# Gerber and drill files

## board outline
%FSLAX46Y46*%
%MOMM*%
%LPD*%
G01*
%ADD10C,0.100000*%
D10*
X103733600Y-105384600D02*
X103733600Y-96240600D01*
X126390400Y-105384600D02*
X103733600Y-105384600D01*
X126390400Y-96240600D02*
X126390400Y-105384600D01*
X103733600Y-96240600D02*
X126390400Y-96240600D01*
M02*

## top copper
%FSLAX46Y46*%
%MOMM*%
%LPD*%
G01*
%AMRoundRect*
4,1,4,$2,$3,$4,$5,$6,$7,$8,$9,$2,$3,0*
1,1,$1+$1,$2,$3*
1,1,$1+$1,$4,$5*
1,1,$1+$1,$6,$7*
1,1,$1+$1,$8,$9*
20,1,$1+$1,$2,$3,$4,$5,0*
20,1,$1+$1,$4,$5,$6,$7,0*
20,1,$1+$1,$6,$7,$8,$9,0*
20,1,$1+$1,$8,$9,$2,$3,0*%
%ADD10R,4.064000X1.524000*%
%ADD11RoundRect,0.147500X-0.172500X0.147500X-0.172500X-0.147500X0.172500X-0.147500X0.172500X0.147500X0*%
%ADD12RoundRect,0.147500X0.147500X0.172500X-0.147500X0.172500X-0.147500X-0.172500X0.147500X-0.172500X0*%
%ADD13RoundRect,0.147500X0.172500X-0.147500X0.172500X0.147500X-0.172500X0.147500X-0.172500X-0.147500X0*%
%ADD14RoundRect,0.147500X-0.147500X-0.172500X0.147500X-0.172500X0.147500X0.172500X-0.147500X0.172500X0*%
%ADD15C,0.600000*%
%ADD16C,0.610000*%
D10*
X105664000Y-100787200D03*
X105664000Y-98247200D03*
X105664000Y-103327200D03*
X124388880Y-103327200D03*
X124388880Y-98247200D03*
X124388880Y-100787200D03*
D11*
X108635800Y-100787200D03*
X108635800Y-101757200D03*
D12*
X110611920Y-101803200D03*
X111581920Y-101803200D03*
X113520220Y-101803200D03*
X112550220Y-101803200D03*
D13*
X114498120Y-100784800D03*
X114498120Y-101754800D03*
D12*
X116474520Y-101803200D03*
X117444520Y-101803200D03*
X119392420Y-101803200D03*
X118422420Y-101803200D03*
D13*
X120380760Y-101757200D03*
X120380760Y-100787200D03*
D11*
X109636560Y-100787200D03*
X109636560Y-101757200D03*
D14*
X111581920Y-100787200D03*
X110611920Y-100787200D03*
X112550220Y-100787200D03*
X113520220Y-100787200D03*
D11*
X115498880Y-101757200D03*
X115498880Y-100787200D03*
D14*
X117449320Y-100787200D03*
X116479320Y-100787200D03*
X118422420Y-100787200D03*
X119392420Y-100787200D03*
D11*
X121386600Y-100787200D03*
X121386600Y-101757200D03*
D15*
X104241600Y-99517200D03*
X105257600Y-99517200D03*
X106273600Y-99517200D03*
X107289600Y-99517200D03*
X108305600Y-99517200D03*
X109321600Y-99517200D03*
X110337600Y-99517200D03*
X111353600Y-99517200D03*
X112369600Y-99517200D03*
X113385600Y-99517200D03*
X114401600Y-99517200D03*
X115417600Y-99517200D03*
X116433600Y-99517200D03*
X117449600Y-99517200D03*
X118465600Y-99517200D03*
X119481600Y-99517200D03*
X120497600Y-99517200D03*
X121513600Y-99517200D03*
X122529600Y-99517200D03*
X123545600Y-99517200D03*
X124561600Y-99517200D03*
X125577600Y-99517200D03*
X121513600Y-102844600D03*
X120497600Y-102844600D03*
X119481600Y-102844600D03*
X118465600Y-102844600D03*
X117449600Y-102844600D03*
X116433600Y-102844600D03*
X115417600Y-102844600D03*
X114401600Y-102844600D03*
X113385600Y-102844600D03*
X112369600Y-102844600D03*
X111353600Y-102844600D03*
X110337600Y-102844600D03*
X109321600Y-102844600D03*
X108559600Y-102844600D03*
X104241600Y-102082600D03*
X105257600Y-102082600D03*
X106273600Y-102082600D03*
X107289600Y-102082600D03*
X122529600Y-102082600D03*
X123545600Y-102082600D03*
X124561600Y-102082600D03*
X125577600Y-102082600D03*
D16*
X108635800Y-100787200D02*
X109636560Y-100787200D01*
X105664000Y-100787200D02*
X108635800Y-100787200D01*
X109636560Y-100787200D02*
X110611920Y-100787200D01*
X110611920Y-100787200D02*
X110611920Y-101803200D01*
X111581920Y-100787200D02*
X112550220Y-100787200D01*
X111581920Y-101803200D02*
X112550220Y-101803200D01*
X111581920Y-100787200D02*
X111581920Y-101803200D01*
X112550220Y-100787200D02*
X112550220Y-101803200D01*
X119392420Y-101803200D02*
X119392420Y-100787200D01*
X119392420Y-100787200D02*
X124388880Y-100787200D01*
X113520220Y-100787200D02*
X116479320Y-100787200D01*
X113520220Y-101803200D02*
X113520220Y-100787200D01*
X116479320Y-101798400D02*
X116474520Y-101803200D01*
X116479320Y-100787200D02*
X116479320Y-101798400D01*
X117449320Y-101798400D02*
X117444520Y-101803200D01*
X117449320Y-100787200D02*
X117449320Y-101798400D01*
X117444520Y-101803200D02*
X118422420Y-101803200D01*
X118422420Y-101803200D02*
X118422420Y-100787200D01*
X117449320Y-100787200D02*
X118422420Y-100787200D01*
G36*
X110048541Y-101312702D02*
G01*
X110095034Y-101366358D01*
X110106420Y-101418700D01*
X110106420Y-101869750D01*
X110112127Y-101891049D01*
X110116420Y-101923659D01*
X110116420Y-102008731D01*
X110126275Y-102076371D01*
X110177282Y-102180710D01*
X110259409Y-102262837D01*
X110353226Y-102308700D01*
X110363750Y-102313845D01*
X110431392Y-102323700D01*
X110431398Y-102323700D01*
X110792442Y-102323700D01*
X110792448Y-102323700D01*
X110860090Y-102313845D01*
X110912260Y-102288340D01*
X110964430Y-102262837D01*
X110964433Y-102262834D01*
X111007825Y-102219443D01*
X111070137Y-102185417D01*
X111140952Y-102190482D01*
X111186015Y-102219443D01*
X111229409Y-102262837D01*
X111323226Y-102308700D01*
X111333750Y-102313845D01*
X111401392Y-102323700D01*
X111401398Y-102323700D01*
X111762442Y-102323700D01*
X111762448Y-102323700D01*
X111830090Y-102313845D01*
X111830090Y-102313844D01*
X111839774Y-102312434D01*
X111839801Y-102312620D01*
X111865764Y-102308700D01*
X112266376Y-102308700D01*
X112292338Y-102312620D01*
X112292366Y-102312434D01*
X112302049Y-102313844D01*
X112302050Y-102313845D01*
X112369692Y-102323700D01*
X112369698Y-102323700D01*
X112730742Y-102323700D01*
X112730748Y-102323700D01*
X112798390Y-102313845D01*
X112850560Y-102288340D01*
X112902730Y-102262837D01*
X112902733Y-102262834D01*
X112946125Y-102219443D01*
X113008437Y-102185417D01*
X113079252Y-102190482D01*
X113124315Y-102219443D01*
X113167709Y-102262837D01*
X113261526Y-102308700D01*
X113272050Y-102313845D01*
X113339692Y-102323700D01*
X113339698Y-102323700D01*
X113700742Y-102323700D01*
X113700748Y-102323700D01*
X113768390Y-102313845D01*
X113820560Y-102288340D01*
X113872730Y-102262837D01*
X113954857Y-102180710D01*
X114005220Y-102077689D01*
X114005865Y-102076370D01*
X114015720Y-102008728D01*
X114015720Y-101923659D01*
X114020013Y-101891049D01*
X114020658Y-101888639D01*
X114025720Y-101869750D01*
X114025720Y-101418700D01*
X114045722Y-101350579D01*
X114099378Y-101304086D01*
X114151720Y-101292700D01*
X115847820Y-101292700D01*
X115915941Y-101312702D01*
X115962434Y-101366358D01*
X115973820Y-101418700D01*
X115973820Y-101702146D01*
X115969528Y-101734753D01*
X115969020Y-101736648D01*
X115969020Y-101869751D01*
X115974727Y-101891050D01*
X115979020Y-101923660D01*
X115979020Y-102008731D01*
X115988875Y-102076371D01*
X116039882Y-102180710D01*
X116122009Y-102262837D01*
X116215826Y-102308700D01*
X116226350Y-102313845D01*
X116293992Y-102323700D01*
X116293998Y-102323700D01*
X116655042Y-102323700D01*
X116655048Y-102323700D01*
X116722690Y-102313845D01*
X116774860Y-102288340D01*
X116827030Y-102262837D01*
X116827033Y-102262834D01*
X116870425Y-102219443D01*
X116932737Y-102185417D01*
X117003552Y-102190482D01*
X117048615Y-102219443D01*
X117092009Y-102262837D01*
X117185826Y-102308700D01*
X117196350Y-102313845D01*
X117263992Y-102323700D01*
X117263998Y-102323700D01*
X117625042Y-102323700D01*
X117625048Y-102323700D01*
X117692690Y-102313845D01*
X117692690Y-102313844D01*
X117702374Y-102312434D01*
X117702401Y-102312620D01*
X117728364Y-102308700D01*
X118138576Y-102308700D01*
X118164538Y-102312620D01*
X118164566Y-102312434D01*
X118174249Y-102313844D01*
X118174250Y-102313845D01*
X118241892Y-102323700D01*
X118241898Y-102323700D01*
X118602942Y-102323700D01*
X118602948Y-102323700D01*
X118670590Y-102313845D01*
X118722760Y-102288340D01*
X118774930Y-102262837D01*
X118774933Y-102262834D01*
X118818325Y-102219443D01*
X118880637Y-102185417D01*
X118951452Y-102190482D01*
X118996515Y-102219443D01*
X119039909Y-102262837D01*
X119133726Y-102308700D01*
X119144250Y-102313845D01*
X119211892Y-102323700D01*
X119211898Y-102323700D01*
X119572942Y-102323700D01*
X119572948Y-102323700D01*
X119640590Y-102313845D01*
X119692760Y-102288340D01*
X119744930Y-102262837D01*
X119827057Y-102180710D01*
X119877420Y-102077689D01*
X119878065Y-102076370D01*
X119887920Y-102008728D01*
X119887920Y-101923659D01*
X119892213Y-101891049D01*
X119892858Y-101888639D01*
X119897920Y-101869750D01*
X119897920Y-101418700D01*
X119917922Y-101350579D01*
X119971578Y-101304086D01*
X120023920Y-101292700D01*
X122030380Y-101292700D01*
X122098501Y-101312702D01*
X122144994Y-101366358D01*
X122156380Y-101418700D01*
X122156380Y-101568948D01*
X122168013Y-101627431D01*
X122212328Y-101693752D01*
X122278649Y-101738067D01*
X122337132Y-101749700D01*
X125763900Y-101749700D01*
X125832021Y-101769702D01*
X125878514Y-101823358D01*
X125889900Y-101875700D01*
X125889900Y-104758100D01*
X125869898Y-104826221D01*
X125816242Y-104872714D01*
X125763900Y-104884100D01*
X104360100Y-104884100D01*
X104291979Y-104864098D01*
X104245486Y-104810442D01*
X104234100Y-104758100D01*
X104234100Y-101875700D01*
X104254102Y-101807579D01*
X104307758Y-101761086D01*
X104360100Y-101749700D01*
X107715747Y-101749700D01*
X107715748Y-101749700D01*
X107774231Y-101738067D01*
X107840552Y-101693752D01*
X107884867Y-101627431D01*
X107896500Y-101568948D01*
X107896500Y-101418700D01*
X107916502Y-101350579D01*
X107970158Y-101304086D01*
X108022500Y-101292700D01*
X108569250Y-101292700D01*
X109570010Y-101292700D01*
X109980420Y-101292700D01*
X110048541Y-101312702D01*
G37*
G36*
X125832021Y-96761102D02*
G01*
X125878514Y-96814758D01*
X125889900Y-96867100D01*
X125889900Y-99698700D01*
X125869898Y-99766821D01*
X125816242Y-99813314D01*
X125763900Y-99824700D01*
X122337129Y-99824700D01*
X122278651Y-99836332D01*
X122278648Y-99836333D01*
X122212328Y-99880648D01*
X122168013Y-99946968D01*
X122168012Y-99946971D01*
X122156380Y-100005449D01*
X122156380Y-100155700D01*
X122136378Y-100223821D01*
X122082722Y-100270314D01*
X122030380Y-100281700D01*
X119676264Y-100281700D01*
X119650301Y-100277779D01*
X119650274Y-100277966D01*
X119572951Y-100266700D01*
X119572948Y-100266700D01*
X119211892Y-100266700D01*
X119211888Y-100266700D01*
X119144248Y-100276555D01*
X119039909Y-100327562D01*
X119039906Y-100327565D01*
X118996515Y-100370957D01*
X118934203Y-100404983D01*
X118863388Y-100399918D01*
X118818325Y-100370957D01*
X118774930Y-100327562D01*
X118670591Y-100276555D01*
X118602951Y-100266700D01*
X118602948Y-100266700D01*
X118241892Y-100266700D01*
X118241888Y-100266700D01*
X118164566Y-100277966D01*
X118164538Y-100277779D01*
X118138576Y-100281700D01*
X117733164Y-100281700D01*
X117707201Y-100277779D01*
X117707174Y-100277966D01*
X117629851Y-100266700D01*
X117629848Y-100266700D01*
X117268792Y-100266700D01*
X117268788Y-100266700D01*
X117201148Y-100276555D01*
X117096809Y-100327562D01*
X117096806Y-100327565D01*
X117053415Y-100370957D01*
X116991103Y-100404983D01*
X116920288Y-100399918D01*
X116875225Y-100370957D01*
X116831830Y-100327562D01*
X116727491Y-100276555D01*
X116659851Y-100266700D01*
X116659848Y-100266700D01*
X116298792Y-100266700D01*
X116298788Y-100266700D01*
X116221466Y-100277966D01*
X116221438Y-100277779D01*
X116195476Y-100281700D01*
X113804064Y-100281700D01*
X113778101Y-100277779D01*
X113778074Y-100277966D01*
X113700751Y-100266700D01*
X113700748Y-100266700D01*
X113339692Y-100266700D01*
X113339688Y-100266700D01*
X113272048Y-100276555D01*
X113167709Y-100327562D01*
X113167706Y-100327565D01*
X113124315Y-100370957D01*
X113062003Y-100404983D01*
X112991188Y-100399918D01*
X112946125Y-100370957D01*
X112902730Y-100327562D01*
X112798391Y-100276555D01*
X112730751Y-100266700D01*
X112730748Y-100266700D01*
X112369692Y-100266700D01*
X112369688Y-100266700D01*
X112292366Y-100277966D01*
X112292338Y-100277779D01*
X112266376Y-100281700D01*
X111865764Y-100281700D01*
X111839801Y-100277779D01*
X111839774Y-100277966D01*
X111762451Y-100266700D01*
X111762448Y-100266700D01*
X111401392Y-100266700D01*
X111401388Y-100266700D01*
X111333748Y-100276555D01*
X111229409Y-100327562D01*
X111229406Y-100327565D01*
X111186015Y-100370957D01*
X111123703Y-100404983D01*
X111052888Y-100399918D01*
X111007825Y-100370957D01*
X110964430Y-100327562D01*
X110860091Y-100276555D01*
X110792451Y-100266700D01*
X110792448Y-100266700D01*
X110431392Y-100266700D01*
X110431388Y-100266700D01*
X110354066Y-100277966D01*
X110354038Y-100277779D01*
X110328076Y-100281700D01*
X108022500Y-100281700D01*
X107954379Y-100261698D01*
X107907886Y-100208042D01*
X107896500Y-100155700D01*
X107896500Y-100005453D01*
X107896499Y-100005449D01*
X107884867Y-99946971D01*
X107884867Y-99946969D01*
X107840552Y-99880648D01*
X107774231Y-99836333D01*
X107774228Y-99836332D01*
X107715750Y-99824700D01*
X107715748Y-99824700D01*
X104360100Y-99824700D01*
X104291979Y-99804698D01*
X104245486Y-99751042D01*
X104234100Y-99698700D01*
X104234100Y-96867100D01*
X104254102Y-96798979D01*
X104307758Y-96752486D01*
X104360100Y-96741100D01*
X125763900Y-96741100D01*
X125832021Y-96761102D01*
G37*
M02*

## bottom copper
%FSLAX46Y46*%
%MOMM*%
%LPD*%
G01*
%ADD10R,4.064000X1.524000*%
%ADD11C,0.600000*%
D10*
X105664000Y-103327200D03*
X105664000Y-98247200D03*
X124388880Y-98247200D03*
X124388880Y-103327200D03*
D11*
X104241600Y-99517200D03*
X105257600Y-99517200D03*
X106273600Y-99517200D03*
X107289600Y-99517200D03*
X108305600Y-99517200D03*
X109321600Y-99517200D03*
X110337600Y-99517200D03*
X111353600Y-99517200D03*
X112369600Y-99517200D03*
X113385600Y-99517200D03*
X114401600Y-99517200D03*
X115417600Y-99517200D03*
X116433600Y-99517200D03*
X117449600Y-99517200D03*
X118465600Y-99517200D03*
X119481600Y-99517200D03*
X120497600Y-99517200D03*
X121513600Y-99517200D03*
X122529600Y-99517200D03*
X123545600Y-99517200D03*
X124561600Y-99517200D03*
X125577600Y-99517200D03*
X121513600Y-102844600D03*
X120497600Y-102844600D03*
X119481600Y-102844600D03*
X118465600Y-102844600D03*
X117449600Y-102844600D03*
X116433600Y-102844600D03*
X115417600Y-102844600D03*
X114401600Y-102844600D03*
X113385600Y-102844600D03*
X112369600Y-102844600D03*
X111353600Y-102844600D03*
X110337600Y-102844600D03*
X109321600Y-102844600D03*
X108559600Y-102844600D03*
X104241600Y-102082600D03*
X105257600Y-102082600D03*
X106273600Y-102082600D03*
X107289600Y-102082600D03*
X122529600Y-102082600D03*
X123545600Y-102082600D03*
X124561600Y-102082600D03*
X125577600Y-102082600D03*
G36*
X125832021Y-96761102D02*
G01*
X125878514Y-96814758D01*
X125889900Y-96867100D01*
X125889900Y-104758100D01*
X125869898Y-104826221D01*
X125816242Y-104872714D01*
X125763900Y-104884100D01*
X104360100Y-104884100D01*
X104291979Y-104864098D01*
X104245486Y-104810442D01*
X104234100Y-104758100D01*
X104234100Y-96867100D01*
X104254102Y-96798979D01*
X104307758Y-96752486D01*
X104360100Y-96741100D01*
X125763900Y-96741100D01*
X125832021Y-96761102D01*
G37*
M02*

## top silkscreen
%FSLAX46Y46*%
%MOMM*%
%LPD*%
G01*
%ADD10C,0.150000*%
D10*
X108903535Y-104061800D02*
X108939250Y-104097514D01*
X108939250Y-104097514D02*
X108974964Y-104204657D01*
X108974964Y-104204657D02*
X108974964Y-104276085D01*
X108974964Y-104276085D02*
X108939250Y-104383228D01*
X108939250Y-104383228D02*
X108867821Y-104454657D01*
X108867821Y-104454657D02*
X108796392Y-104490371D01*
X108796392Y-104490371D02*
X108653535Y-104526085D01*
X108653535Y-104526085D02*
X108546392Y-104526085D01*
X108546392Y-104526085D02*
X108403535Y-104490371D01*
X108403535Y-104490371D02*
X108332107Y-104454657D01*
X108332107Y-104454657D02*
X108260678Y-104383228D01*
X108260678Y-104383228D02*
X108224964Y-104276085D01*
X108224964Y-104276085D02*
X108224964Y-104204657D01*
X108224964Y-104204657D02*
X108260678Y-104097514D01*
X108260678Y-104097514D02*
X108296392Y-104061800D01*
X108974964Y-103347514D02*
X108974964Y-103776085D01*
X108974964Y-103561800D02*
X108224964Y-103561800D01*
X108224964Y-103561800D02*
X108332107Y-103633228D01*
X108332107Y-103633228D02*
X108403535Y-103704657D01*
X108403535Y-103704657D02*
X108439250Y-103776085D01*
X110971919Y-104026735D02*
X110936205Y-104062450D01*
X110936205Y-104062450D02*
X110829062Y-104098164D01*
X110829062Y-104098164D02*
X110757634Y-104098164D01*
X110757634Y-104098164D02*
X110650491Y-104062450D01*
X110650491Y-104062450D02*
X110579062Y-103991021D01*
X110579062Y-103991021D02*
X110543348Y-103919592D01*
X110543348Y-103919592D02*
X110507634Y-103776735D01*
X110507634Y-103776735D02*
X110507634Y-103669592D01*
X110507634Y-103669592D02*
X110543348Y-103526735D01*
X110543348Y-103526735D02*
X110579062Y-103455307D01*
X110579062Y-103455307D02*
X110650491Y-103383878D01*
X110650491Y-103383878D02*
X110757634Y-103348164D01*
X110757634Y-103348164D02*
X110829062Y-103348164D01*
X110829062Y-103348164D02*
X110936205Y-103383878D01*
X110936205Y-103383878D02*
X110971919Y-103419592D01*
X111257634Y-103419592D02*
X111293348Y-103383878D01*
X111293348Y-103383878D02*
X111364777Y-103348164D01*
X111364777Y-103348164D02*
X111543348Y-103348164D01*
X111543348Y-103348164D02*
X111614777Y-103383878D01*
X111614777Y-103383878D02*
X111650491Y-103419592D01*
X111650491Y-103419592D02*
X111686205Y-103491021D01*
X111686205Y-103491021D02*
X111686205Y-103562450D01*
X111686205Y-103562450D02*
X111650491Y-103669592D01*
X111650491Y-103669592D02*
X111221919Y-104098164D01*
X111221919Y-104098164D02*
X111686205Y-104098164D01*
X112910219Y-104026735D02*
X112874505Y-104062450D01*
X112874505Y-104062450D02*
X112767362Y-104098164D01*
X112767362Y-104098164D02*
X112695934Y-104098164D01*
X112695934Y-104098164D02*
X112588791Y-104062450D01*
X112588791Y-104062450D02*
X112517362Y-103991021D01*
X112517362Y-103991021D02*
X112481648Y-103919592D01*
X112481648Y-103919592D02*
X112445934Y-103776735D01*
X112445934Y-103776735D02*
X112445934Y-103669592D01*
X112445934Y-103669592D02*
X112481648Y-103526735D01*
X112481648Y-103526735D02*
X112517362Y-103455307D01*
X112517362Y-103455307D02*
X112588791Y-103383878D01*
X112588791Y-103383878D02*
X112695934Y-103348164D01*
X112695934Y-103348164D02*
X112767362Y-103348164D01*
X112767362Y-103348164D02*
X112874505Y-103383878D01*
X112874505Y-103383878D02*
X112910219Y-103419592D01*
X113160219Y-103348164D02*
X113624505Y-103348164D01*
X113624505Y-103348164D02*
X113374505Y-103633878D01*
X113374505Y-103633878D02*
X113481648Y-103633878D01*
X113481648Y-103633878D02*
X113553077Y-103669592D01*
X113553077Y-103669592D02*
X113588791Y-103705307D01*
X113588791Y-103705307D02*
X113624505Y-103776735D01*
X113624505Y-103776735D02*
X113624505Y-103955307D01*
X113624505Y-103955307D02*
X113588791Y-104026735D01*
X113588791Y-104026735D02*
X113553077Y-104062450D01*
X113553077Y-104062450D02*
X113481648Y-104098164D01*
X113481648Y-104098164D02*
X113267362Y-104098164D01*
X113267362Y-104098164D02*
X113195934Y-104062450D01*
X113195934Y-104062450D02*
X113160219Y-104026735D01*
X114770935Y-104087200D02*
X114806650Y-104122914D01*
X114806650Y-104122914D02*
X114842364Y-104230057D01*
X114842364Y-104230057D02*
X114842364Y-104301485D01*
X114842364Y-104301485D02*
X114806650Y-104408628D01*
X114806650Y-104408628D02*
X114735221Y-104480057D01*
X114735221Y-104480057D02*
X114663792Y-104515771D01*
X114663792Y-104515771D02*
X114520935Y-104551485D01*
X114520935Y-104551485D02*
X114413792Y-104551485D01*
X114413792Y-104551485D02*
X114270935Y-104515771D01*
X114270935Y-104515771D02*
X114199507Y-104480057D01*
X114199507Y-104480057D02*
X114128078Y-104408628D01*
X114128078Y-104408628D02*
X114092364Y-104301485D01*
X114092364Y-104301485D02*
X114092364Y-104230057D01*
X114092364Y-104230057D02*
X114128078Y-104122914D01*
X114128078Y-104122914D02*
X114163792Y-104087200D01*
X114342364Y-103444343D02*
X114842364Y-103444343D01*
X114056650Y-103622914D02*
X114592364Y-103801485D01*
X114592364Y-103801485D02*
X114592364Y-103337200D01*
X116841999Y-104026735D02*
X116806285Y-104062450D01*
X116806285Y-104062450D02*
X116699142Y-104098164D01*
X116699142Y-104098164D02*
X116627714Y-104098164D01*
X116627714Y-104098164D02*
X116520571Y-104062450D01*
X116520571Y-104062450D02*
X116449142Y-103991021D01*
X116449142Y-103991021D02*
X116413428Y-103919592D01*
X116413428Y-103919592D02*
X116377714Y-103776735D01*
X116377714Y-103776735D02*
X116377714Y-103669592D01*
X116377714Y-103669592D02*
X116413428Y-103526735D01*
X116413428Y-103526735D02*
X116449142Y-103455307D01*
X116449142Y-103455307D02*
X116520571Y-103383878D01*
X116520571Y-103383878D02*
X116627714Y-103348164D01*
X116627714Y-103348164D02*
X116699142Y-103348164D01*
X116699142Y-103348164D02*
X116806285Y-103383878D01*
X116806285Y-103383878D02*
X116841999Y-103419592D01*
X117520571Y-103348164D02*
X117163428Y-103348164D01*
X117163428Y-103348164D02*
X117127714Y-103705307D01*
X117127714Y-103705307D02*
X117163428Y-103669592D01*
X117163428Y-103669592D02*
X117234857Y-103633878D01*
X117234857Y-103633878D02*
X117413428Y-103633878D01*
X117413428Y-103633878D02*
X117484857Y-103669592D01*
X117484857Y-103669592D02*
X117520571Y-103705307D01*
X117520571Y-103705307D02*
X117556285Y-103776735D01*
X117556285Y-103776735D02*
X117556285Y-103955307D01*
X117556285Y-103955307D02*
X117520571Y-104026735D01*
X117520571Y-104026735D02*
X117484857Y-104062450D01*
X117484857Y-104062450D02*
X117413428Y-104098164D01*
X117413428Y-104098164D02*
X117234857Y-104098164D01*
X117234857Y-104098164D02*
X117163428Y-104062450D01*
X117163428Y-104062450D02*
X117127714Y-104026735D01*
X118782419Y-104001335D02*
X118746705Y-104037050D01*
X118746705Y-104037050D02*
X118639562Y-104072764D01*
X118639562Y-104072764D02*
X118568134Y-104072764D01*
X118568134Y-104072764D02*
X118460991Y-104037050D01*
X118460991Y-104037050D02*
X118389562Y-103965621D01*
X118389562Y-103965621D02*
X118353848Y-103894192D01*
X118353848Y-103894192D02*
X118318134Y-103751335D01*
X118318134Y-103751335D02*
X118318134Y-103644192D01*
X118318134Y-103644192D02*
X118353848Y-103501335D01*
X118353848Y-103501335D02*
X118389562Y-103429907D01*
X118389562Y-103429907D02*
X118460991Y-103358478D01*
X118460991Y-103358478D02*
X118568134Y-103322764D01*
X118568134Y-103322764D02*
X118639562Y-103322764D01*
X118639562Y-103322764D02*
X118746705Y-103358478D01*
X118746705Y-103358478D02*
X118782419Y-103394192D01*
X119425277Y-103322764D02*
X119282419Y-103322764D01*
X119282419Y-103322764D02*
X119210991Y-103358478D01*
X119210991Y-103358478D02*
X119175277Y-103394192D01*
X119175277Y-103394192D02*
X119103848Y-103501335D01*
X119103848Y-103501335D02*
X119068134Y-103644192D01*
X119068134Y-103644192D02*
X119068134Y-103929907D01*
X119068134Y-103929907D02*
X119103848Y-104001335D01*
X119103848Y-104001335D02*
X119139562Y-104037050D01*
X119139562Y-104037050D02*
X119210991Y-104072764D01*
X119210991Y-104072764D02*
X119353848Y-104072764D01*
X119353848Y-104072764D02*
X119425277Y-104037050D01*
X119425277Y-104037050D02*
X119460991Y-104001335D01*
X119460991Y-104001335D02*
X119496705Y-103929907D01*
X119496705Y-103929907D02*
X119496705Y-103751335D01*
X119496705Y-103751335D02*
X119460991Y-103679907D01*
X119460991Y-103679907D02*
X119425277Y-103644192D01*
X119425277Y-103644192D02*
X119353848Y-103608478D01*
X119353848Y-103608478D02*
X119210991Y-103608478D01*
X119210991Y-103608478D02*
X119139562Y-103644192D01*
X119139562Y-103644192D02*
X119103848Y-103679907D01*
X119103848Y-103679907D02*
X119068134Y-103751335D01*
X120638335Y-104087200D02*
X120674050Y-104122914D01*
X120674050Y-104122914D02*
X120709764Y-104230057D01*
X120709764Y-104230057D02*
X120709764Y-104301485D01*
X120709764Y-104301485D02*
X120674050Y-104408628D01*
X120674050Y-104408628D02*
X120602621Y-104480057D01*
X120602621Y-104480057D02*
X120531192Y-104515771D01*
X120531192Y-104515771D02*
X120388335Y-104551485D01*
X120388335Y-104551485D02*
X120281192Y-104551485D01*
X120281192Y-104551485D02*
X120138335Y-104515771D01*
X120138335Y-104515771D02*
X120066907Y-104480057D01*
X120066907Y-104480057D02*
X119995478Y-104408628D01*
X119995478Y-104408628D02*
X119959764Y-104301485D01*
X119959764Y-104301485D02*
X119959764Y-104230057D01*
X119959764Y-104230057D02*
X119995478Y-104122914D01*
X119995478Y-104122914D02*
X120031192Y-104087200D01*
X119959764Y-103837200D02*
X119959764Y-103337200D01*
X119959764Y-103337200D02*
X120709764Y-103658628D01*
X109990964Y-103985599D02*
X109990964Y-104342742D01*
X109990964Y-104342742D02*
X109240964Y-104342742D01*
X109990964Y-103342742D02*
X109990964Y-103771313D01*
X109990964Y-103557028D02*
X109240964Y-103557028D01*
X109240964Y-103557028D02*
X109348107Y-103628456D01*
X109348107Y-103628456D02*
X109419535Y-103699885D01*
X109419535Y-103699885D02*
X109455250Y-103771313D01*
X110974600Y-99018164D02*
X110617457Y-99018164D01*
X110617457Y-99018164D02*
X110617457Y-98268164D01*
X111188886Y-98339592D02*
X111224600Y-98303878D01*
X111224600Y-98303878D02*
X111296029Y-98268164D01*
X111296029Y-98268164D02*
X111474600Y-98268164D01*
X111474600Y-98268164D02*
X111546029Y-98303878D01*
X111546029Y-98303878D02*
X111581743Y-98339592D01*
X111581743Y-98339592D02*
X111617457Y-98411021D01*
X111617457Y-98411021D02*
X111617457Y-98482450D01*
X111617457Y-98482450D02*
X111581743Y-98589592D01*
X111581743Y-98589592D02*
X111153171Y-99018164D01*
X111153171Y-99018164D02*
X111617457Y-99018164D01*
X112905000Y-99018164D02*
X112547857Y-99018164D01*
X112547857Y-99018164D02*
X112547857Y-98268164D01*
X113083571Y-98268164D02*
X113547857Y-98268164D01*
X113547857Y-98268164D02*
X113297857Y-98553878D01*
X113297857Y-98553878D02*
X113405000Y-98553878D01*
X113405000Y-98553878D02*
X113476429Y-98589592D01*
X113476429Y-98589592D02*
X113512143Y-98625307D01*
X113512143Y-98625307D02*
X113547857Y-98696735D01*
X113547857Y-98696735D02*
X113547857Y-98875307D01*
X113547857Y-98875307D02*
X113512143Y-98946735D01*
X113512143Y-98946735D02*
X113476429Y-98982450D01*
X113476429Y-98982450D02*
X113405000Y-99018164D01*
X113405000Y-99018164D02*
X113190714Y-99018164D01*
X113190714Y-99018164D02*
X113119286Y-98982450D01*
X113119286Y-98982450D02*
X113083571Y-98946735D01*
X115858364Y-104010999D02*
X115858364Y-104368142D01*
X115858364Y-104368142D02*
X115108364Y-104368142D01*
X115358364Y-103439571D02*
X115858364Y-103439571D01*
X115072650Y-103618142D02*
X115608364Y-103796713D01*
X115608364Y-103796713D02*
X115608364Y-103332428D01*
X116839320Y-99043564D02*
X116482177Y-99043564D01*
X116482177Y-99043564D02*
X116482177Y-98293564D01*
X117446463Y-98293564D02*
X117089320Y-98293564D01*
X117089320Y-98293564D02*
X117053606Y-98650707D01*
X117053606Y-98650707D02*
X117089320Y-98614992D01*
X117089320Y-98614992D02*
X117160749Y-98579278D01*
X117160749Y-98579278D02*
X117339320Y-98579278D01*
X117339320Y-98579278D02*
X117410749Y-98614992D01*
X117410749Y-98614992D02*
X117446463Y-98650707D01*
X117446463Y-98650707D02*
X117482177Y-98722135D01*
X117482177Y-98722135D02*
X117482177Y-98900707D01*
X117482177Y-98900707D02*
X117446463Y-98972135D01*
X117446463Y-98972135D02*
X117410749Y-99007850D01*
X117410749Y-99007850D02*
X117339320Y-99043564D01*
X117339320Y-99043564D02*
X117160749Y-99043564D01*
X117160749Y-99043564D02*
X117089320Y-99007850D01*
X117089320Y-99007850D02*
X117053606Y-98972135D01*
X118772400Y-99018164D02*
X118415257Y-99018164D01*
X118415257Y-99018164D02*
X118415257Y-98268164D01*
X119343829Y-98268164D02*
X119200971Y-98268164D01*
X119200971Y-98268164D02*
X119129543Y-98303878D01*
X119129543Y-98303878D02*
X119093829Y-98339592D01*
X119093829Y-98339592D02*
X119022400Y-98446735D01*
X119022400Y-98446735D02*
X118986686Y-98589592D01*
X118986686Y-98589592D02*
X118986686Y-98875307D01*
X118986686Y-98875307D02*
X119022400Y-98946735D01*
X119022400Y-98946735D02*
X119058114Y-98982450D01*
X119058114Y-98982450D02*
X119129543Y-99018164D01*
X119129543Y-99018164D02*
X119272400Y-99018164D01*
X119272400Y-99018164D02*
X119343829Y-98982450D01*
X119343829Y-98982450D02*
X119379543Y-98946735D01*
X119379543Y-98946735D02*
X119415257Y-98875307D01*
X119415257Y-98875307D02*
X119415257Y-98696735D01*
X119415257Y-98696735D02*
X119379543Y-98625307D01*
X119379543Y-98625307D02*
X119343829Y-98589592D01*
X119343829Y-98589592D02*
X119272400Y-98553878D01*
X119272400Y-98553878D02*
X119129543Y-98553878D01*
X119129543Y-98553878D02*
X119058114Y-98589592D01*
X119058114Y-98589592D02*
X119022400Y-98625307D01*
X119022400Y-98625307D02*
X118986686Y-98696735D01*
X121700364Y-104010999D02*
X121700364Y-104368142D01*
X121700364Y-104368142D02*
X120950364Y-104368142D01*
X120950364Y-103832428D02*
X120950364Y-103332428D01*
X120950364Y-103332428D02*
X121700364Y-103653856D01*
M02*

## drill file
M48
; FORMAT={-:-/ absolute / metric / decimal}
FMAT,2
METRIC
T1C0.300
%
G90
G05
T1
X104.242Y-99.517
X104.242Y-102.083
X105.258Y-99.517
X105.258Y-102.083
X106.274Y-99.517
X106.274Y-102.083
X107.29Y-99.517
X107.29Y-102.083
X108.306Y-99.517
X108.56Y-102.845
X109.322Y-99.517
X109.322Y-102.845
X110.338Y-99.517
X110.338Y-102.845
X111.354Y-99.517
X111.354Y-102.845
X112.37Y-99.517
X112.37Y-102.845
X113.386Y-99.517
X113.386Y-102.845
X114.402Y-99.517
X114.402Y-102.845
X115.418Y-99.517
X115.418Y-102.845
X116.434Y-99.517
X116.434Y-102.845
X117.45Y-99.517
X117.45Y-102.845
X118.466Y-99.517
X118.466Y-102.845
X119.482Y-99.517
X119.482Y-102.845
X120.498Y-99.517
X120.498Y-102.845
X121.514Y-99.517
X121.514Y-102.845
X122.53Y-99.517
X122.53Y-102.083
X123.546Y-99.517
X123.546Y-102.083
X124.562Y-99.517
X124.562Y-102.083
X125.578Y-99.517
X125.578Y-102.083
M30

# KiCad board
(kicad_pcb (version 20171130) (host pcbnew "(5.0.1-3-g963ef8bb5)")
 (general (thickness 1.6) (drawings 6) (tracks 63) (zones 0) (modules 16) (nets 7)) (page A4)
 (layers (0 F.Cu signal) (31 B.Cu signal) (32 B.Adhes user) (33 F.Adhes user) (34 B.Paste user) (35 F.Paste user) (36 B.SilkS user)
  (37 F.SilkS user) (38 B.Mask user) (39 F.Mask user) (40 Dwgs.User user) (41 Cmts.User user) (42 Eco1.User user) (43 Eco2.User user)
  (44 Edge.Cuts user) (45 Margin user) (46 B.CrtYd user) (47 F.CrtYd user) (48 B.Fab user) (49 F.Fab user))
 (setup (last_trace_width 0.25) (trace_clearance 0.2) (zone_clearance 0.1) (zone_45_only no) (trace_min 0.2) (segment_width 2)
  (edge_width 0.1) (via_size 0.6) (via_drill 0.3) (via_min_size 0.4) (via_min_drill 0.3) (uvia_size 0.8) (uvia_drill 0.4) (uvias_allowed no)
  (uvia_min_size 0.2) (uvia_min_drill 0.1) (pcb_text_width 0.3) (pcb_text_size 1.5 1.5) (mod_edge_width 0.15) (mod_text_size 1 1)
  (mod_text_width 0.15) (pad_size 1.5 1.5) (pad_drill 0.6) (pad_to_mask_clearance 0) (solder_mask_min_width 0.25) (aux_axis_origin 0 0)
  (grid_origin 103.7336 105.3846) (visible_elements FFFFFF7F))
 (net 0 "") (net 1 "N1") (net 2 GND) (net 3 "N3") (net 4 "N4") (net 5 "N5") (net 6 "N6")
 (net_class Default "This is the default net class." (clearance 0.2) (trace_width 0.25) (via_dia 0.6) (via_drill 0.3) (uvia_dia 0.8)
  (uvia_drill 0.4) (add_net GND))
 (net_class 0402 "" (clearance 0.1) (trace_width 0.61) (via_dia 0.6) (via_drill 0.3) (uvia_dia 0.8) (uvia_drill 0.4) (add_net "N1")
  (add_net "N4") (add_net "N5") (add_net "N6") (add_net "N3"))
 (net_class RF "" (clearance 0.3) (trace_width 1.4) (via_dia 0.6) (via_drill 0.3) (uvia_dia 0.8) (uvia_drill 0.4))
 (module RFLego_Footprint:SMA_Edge (layer F.Cu) (at 103.632 100.7872)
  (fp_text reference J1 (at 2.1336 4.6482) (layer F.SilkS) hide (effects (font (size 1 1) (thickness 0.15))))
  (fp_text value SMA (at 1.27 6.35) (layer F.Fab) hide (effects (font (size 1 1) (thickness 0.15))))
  (pad 1 smd rect (at 2.032 0) (size 4.064 1.524) (layers F.Cu F.Mask) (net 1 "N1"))
  (pad 2 smd rect (at 2.032 -2.54) (size 4.064 1.524) (layers F.Cu F.Mask) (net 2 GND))
  (pad 2 smd rect (at 2.032 2.54) (size 4.064 1.524) (layers B.Cu B.Mask) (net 2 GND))
  (pad 2 smd rect (at 2.032 -2.54) (size 4.064 1.524) (layers B.Cu B.Mask) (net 2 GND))
  (pad 2 smd rect (at 2.032 2.54) (size 4.064 1.524) (layers F.Cu F.Mask) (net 2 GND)))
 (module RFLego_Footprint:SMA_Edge (layer F.Cu) (at 122.35688 100.7872)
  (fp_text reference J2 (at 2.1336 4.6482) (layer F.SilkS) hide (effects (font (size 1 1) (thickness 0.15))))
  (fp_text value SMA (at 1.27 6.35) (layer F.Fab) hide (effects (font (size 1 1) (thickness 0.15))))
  (pad 2 smd rect (at 2.032 2.54) (size 4.064 1.524) (layers F.Cu F.Mask) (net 2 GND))
  (pad 2 smd rect (at 2.032 -2.54) (size 4.064 1.524) (layers B.Cu B.Mask) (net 2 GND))
  (pad 2 smd rect (at 2.032 2.54) (size 4.064 1.524) (layers B.Cu B.Mask) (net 2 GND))
  (pad 2 smd rect (at 2.032 -2.54) (size 4.064 1.524) (layers F.Cu F.Mask) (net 2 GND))
  (pad 1 smd rect (at 2.032 0) (size 4.064 1.524) (layers F.Cu F.Mask) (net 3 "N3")))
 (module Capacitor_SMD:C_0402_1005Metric (layer F.Cu) (at 108.6358 101.2722 270)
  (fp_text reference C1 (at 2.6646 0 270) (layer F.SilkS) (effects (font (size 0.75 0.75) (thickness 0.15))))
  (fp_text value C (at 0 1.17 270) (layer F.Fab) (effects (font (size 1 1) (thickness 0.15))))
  (pad 1 smd roundrect (at -0.485 0 270) (size 0.59 0.64) (layers F.Cu F.Paste F.Mask) (roundrect_rratio 0.25) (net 1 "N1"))
  (pad 2 smd roundrect (at 0.485 0 270) (size 0.59 0.64) (layers F.Cu F.Paste F.Mask) (roundrect_rratio 0.25) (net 2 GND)))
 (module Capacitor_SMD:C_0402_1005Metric (layer F.Cu) (at 111.09692 101.8032 180)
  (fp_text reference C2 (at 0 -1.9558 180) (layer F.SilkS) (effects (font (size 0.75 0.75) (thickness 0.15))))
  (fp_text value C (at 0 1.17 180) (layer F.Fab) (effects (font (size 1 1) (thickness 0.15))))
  (pad 2 smd roundrect (at 0.485 0 180) (size 0.59 0.64) (layers F.Cu F.Paste F.Mask) (roundrect_rratio 0.25) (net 1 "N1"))
  (pad 1 smd roundrect (at -0.485 0 180) (size 0.59 0.64) (layers F.Cu F.Paste F.Mask) (roundrect_rratio 0.25) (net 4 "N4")))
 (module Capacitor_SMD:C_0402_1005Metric (layer F.Cu) (at 113.03522 101.8032 180)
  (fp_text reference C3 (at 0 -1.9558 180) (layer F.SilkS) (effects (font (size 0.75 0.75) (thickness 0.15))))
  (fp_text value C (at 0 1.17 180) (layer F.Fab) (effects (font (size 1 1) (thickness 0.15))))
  (pad 1 smd roundrect (at -0.485 0 180) (size 0.59 0.64) (layers F.Cu F.Paste F.Mask) (roundrect_rratio 0.25) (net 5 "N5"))
  (pad 2 smd roundrect (at 0.485 0 180) (size 0.59 0.64) (layers F.Cu F.Paste F.Mask) (roundrect_rratio 0.25) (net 4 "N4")))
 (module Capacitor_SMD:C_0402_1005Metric (layer F.Cu) (at 114.49812 101.2698 90)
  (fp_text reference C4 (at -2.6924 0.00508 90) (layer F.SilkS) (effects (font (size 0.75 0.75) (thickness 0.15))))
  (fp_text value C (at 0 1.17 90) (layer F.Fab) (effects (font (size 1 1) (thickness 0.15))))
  (pad 2 smd roundrect (at 0.485 0 90) (size 0.59 0.64) (layers F.Cu F.Paste F.Mask) (roundrect_rratio 0.25) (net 5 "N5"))
  (pad 1 smd roundrect (at -0.485 0 90) (size 0.59 0.64) (layers F.Cu F.Paste F.Mask) (roundrect_rratio 0.25) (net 2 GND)))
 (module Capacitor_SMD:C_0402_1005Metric (layer F.Cu) (at 116.95952 101.8032 180)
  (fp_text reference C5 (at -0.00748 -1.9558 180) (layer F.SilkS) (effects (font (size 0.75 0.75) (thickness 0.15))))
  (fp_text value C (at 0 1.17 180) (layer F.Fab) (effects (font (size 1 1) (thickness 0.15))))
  (pad 2 smd roundrect (at 0.485 0 180) (size 0.59 0.64) (layers F.Cu F.Paste F.Mask) (roundrect_rratio 0.25) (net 5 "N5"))
  (pad 1 smd roundrect (at -0.485 0 180) (size 0.59 0.64) (layers F.Cu F.Paste F.Mask) (roundrect_rratio 0.25) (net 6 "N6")))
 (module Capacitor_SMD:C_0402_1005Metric (layer F.Cu) (at 118.90742 101.8032 180)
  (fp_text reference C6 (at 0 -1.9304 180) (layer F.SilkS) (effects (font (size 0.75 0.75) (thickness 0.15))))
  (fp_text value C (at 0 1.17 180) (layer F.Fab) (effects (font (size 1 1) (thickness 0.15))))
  (pad 1 smd roundrect (at -0.485 0 180) (size 0.59 0.64) (layers F.Cu F.Paste F.Mask) (roundrect_rratio 0.25) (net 3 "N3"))
  (pad 2 smd roundrect (at 0.485 0 180) (size 0.59 0.64) (layers F.Cu F.Paste F.Mask) (roundrect_rratio 0.25) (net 6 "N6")))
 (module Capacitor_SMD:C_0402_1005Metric (layer F.Cu) (at 120.38076 101.2722 90)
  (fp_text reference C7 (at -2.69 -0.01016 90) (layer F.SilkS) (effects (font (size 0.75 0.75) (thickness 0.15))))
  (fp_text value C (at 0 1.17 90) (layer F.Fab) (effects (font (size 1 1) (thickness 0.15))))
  (pad 1 smd roundrect (at -0.485 0 90) (size 0.59 0.64) (layers F.Cu F.Paste F.Mask) (roundrect_rratio 0.25) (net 2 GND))
  (pad 2 smd roundrect (at 0.485 0 90) (size 0.59 0.64) (layers F.Cu F.Paste F.Mask) (roundrect_rratio 0.25) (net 3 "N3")))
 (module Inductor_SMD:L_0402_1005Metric (layer F.Cu) (at 109.63656 101.2722 270)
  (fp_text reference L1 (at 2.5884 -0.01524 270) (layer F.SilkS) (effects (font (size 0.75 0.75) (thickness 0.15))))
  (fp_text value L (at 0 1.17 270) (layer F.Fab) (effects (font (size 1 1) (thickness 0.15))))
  (pad 1 smd roundrect (at -0.485 0 270) (size 0.59 0.64) (layers F.Cu F.Paste F.Mask) (roundrect_rratio 0.25) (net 1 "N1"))
  (pad 2 smd roundrect (at 0.485 0 270) (size 0.59 0.64) (layers F.Cu F.Paste F.Mask) (roundrect_rratio 0.25) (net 2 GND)))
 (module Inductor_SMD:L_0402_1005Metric (layer F.Cu) (at 111.09692 100.7872)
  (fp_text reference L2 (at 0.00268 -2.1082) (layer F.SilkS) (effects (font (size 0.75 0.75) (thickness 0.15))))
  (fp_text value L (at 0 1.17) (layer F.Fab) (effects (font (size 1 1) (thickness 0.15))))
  (pad 2 smd roundrect (at 0.485 0) (size 0.59 0.64) (layers F.Cu F.Paste F.Mask) (roundrect_rratio 0.25) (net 4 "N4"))
  (pad 1 smd roundrect (at -0.485 0) (size 0.59 0.64) (layers F.Cu F.Paste F.Mask) (roundrect_rratio 0.25) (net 1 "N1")))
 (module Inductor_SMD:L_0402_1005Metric (layer F.Cu) (at 113.03522 100.7872)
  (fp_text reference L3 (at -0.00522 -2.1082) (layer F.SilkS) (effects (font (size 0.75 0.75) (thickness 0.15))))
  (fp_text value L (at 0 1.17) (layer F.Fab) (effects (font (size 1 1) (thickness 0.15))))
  (pad 1 smd roundrect (at -0.485 0) (size 0.59 0.64) (layers F.Cu F.Paste F.Mask) (roundrect_rratio 0.25) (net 4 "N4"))
  (pad 2 smd roundrect (at 0.485 0) (size 0.59 0.64) (layers F.Cu F.Paste F.Mask) (roundrect_rratio 0.25) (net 5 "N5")))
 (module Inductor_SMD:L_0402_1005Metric (layer F.Cu) (at 115.49888 101.2722 270)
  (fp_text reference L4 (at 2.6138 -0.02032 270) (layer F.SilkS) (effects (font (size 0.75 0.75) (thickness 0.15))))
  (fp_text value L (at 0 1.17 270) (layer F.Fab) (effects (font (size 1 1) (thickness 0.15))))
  (pad 2 smd roundrect (at 0.485 0 270) (size 0.59 0.64) (layers F.Cu F.Paste F.Mask) (roundrect_rratio 0.25) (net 2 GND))
  (pad 1 smd roundrect (at -0.485 0 270) (size 0.59 0.64) (layers F.Cu F.Paste F.Mask) (roundrect_rratio 0.25) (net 5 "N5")))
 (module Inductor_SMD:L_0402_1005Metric (layer F.Cu) (at 116.96432 100.7872)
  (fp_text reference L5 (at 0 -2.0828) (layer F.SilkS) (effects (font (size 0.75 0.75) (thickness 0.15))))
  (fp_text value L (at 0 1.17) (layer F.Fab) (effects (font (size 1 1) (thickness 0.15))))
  (pad 2 smd roundrect (at 0.485 0) (size 0.59 0.64) (layers F.Cu F.Paste F.Mask) (roundrect_rratio 0.25) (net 6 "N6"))
  (pad 1 smd roundrect (at -0.485 0) (size 0.59 0.64) (layers F.Cu F.Paste F.Mask) (roundrect_rratio 0.25) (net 5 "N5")))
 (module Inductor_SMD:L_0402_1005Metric (layer F.Cu) (at 118.90742 100.7872)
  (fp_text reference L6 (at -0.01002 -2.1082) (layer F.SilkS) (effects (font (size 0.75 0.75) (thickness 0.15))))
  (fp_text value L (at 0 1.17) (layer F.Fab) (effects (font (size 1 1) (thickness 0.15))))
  (pad 1 smd roundrect (at -0.485 0) (size 0.59 0.64) (layers F.Cu F.Paste F.Mask) (roundrect_rratio 0.25) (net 6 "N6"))
  (pad 2 smd roundrect (at 0.485 0) (size 0.59 0.64) (layers F.Cu F.Paste F.Mask) (roundrect_rratio 0.25) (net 3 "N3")))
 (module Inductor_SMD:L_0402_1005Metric (layer F.Cu) (at 121.3866 101.2722 270)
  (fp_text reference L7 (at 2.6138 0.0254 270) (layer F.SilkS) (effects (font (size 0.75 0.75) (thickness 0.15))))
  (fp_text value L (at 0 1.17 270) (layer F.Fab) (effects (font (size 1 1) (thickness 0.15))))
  (pad 1 smd roundrect (at -0.485 0 270) (size 0.59 0.64) (layers F.Cu F.Paste F.Mask) (roundrect_rratio 0.25) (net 3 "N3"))
  (pad 2 smd roundrect (at 0.485 0 270) (size 0.59 0.64) (layers F.Cu F.Paste F.Mask) (roundrect_rratio 0.25) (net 2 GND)))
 (gr_line (start 103.7336 105.3846) (end 103.7336 96.2406) (layer Edge.Cuts) (width 0.1))
 (gr_line (start 126.3904 105.3846) (end 103.7336 105.3846) (layer Edge.Cuts) (width 0.1))
 (gr_line (start 126.3904 96.2406) (end 126.3904 105.3846) (layer Edge.Cuts) (width 0.1))
 (gr_line (start 103.7336 96.2406) (end 126.3904 96.2406) (layer Edge.Cuts) (width 0.1))
 (segment (start 108.6358 100.7872) (end 109.63656 100.7872) (width 0.61) (layer F.Cu) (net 1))
 (segment (start 105.664 100.7872) (end 108.6358 100.7872) (width 0.61) (layer F.Cu) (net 1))
 (segment (start 109.63656 100.7872) (end 110.61192 100.7872) (width 0.61) (layer F.Cu) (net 1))
 (segment (start 110.61192 100.7872) (end 110.61192 101.8032) (width 0.61) (layer F.Cu) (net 1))
 (segment (start 111.58192 100.7872) (end 112.55022 100.7872) (width 0.61) (layer F.Cu) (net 4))
 (segment (start 111.58192 101.8032) (end 112.55022 101.8032) (width 0.61) (layer F.Cu) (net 4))
 (segment (start 111.58192 100.7872) (end 111.58192 101.8032) (width 0.61) (layer F.Cu) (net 4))
 (segment (start 112.55022 100.7872) (end 112.55022 101.8032) (width 0.61) (layer F.Cu) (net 4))
 (segment (start 119.39242 101.8032) (end 119.39242 100.7872) (width 0.61) (layer F.Cu) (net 3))
 (segment (start 119.39242 100.7872) (end 124.38888 100.7872) (width 0.61) (layer F.Cu) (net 3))
 (via (at 104.2416 99.5172) (size 0.6) (drill 0.3) (layers F.Cu B.Cu) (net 2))
 (via (at 105.2576 99.5172) (size 0.6) (drill 0.3) (layers F.Cu B.Cu) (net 2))
 (via (at 106.2736 99.5172) (size 0.6) (drill 0.3) (layers F.Cu B.Cu) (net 2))
 (via (at 107.2896 99.5172) (size 0.6) (drill 0.3) (layers F.Cu B.Cu) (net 2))
 (via (at 108.3056 99.5172) (size 0.6) (drill 0.3) (layers F.Cu B.Cu) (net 2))
 (via (at 109.3216 99.5172) (size 0.6) (drill 0.3) (layers F.Cu B.Cu) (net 2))
 (via (at 110.3376 99.5172) (size 0.6) (drill 0.3) (layers F.Cu B.Cu) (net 2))
 (via (at 111.3536 99.5172) (size 0.6) (drill 0.3) (layers F.Cu B.Cu) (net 2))
 (via (at 112.3696 99.5172) (size 0.6) (drill 0.3) (layers F.Cu B.Cu) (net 2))
 (via (at 113.3856 99.5172) (size 0.6) (drill 0.3) (layers F.Cu B.Cu) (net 2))
 (via (at 114.4016 99.5172) (size 0.6) (drill 0.3) (layers F.Cu B.Cu) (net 2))
 (via (at 115.4176 99.5172) (size 0.6) (drill 0.3) (layers F.Cu B.Cu) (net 2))
 (via (at 116.4336 99.5172) (size 0.6) (drill 0.3) (layers F.Cu B.Cu) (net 2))
 (via (at 117.4496 99.5172) (size 0.6) (drill 0.3) (layers F.Cu B.Cu) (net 2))
 (via (at 118.4656 99.5172) (size 0.6) (drill 0.3) (layers F.Cu B.Cu) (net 2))
 (via (at 119.4816 99.5172) (size 0.6) (drill 0.3) (layers F.Cu B.Cu) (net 2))
 (via (at 120.4976 99.5172) (size 0.6) (drill 0.3) (layers F.Cu B.Cu) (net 2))
 (via (at 121.5136 99.5172) (size 0.6) (drill 0.3) (layers F.Cu B.Cu) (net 2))
 (via (at 122.5296 99.5172) (size 0.6) (drill 0.3) (layers F.Cu B.Cu) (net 2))
 (via (at 123.5456 99.5172) (size 0.6) (drill 0.3) (layers F.Cu B.Cu) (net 2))
 (via (at 124.5616 99.5172) (size 0.6) (drill 0.3) (layers F.Cu B.Cu) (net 2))
 (via (at 125.5776 99.5172) (size 0.6) (drill 0.3) (layers F.Cu B.Cu) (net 2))
 (via (at 121.5136 102.8446) (size 0.6) (drill 0.3) (layers F.Cu B.Cu) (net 2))
 (via (at 120.4976 102.8446) (size 0.6) (drill 0.3) (layers F.Cu B.Cu) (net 2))
 (via (at 119.4816 102.8446) (size 0.6) (drill 0.3) (layers F.Cu B.Cu) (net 2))
 (via (at 118.4656 102.8446) (size 0.6) (drill 0.3) (layers F.Cu B.Cu) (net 2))
 (via (at 117.4496 102.8446) (size 0.6) (drill 0.3) (layers F.Cu B.Cu) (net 2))
 (via (at 116.4336 102.8446) (size 0.6) (drill 0.3) (layers F.Cu B.Cu) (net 2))
 (via (at 115.4176 102.8446) (size 0.6) (drill 0.3) (layers F.Cu B.Cu) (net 2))
 (via (at 114.4016 102.8446) (size 0.6) (drill 0.3) (layers F.Cu B.Cu) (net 2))
 (via (at 113.3856 102.8446) (size 0.6) (drill 0.3) (layers F.Cu B.Cu) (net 2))
 (via (at 112.3696 102.8446) (size 0.6) (drill 0.3) (layers F.Cu B.Cu) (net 2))
 (via (at 111.3536 102.8446) (size 0.6) (drill 0.3) (layers F.Cu B.Cu) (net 2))
 (via (at 110.3376 102.8446) (size 0.6) (drill 0.3) (layers F.Cu B.Cu) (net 2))
 (via (at 109.3216 102.8446) (size 0.6) (drill 0.3) (layers F.Cu B.Cu) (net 2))
 (via (at 108.5596 102.8446) (size 0.6) (drill 0.3) (layers F.Cu B.Cu) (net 2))
 (via (at 104.2416 102.0826) (size 0.6) (drill 0.3) (layers F.Cu B.Cu) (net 2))
 (via (at 105.2576 102.0826) (size 0.6) (drill 0.3) (layers F.Cu B.Cu) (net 2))
 (via (at 106.2736 102.0826) (size 0.6) (drill 0.3) (layers F.Cu B.Cu) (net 2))
 (via (at 107.2896 102.0826) (size 0.6) (drill 0.3) (layers F.Cu B.Cu) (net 2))
 (via (at 122.5296 102.0826) (size 0.6) (drill 0.3) (layers F.Cu B.Cu) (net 2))
 (via (at 123.5456 102.0826) (size 0.6) (drill 0.3) (layers F.Cu B.Cu) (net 2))
 (via (at 124.5616 102.0826) (size 0.6) (drill 0.3) (layers F.Cu B.Cu) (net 2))
 (via (at 125.5776 102.0826) (size 0.6) (drill 0.3) (layers F.Cu B.Cu) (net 2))
 (segment (start 113.52022 100.7872) (end 116.47932 100.7872) (width 0.61) (layer F.Cu) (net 5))
 (segment (start 113.52022 101.8032) (end 113.52022 100.7872) (width 0.61) (layer F.Cu) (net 5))
 (segment (start 116.47932 101.7984) (end 116.47452 101.8032) (width 0.61) (layer F.Cu) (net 5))
 (segment (start 116.47932 100.7872) (end 116.47932 101.7984) (width 0.61) (layer F.Cu) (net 5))
 (segment (start 117.44932 101.7984) (end 117.44452 101.8032) (width 0.61) (layer F.Cu) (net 6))
 (segment (start 117.44932 100.7872) (end 117.44932 101.7984) (width 0.61) (layer F.Cu) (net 6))
 (segment (start 117.44452 101.8032) (end 118.42242 101.8032) (width 0.61) (layer F.Cu) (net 6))
 (segment (start 118.42242 101.8032) (end 118.42242 100.7872) (width 0.61) (layer F.Cu) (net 6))
 (segment (start 117.44932 100.7872) (end 118.42242 100.7872) (width 0.61) (layer F.Cu) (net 6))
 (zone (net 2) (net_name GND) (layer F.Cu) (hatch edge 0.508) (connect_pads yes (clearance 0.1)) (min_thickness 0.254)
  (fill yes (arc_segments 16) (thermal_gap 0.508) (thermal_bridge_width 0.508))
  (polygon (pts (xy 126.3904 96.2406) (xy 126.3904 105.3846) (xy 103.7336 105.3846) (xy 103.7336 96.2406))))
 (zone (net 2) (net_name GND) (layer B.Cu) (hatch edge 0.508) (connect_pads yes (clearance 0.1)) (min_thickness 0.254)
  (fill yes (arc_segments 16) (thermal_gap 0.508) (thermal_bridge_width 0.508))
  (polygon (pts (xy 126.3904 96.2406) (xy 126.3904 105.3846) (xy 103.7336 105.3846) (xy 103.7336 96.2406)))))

